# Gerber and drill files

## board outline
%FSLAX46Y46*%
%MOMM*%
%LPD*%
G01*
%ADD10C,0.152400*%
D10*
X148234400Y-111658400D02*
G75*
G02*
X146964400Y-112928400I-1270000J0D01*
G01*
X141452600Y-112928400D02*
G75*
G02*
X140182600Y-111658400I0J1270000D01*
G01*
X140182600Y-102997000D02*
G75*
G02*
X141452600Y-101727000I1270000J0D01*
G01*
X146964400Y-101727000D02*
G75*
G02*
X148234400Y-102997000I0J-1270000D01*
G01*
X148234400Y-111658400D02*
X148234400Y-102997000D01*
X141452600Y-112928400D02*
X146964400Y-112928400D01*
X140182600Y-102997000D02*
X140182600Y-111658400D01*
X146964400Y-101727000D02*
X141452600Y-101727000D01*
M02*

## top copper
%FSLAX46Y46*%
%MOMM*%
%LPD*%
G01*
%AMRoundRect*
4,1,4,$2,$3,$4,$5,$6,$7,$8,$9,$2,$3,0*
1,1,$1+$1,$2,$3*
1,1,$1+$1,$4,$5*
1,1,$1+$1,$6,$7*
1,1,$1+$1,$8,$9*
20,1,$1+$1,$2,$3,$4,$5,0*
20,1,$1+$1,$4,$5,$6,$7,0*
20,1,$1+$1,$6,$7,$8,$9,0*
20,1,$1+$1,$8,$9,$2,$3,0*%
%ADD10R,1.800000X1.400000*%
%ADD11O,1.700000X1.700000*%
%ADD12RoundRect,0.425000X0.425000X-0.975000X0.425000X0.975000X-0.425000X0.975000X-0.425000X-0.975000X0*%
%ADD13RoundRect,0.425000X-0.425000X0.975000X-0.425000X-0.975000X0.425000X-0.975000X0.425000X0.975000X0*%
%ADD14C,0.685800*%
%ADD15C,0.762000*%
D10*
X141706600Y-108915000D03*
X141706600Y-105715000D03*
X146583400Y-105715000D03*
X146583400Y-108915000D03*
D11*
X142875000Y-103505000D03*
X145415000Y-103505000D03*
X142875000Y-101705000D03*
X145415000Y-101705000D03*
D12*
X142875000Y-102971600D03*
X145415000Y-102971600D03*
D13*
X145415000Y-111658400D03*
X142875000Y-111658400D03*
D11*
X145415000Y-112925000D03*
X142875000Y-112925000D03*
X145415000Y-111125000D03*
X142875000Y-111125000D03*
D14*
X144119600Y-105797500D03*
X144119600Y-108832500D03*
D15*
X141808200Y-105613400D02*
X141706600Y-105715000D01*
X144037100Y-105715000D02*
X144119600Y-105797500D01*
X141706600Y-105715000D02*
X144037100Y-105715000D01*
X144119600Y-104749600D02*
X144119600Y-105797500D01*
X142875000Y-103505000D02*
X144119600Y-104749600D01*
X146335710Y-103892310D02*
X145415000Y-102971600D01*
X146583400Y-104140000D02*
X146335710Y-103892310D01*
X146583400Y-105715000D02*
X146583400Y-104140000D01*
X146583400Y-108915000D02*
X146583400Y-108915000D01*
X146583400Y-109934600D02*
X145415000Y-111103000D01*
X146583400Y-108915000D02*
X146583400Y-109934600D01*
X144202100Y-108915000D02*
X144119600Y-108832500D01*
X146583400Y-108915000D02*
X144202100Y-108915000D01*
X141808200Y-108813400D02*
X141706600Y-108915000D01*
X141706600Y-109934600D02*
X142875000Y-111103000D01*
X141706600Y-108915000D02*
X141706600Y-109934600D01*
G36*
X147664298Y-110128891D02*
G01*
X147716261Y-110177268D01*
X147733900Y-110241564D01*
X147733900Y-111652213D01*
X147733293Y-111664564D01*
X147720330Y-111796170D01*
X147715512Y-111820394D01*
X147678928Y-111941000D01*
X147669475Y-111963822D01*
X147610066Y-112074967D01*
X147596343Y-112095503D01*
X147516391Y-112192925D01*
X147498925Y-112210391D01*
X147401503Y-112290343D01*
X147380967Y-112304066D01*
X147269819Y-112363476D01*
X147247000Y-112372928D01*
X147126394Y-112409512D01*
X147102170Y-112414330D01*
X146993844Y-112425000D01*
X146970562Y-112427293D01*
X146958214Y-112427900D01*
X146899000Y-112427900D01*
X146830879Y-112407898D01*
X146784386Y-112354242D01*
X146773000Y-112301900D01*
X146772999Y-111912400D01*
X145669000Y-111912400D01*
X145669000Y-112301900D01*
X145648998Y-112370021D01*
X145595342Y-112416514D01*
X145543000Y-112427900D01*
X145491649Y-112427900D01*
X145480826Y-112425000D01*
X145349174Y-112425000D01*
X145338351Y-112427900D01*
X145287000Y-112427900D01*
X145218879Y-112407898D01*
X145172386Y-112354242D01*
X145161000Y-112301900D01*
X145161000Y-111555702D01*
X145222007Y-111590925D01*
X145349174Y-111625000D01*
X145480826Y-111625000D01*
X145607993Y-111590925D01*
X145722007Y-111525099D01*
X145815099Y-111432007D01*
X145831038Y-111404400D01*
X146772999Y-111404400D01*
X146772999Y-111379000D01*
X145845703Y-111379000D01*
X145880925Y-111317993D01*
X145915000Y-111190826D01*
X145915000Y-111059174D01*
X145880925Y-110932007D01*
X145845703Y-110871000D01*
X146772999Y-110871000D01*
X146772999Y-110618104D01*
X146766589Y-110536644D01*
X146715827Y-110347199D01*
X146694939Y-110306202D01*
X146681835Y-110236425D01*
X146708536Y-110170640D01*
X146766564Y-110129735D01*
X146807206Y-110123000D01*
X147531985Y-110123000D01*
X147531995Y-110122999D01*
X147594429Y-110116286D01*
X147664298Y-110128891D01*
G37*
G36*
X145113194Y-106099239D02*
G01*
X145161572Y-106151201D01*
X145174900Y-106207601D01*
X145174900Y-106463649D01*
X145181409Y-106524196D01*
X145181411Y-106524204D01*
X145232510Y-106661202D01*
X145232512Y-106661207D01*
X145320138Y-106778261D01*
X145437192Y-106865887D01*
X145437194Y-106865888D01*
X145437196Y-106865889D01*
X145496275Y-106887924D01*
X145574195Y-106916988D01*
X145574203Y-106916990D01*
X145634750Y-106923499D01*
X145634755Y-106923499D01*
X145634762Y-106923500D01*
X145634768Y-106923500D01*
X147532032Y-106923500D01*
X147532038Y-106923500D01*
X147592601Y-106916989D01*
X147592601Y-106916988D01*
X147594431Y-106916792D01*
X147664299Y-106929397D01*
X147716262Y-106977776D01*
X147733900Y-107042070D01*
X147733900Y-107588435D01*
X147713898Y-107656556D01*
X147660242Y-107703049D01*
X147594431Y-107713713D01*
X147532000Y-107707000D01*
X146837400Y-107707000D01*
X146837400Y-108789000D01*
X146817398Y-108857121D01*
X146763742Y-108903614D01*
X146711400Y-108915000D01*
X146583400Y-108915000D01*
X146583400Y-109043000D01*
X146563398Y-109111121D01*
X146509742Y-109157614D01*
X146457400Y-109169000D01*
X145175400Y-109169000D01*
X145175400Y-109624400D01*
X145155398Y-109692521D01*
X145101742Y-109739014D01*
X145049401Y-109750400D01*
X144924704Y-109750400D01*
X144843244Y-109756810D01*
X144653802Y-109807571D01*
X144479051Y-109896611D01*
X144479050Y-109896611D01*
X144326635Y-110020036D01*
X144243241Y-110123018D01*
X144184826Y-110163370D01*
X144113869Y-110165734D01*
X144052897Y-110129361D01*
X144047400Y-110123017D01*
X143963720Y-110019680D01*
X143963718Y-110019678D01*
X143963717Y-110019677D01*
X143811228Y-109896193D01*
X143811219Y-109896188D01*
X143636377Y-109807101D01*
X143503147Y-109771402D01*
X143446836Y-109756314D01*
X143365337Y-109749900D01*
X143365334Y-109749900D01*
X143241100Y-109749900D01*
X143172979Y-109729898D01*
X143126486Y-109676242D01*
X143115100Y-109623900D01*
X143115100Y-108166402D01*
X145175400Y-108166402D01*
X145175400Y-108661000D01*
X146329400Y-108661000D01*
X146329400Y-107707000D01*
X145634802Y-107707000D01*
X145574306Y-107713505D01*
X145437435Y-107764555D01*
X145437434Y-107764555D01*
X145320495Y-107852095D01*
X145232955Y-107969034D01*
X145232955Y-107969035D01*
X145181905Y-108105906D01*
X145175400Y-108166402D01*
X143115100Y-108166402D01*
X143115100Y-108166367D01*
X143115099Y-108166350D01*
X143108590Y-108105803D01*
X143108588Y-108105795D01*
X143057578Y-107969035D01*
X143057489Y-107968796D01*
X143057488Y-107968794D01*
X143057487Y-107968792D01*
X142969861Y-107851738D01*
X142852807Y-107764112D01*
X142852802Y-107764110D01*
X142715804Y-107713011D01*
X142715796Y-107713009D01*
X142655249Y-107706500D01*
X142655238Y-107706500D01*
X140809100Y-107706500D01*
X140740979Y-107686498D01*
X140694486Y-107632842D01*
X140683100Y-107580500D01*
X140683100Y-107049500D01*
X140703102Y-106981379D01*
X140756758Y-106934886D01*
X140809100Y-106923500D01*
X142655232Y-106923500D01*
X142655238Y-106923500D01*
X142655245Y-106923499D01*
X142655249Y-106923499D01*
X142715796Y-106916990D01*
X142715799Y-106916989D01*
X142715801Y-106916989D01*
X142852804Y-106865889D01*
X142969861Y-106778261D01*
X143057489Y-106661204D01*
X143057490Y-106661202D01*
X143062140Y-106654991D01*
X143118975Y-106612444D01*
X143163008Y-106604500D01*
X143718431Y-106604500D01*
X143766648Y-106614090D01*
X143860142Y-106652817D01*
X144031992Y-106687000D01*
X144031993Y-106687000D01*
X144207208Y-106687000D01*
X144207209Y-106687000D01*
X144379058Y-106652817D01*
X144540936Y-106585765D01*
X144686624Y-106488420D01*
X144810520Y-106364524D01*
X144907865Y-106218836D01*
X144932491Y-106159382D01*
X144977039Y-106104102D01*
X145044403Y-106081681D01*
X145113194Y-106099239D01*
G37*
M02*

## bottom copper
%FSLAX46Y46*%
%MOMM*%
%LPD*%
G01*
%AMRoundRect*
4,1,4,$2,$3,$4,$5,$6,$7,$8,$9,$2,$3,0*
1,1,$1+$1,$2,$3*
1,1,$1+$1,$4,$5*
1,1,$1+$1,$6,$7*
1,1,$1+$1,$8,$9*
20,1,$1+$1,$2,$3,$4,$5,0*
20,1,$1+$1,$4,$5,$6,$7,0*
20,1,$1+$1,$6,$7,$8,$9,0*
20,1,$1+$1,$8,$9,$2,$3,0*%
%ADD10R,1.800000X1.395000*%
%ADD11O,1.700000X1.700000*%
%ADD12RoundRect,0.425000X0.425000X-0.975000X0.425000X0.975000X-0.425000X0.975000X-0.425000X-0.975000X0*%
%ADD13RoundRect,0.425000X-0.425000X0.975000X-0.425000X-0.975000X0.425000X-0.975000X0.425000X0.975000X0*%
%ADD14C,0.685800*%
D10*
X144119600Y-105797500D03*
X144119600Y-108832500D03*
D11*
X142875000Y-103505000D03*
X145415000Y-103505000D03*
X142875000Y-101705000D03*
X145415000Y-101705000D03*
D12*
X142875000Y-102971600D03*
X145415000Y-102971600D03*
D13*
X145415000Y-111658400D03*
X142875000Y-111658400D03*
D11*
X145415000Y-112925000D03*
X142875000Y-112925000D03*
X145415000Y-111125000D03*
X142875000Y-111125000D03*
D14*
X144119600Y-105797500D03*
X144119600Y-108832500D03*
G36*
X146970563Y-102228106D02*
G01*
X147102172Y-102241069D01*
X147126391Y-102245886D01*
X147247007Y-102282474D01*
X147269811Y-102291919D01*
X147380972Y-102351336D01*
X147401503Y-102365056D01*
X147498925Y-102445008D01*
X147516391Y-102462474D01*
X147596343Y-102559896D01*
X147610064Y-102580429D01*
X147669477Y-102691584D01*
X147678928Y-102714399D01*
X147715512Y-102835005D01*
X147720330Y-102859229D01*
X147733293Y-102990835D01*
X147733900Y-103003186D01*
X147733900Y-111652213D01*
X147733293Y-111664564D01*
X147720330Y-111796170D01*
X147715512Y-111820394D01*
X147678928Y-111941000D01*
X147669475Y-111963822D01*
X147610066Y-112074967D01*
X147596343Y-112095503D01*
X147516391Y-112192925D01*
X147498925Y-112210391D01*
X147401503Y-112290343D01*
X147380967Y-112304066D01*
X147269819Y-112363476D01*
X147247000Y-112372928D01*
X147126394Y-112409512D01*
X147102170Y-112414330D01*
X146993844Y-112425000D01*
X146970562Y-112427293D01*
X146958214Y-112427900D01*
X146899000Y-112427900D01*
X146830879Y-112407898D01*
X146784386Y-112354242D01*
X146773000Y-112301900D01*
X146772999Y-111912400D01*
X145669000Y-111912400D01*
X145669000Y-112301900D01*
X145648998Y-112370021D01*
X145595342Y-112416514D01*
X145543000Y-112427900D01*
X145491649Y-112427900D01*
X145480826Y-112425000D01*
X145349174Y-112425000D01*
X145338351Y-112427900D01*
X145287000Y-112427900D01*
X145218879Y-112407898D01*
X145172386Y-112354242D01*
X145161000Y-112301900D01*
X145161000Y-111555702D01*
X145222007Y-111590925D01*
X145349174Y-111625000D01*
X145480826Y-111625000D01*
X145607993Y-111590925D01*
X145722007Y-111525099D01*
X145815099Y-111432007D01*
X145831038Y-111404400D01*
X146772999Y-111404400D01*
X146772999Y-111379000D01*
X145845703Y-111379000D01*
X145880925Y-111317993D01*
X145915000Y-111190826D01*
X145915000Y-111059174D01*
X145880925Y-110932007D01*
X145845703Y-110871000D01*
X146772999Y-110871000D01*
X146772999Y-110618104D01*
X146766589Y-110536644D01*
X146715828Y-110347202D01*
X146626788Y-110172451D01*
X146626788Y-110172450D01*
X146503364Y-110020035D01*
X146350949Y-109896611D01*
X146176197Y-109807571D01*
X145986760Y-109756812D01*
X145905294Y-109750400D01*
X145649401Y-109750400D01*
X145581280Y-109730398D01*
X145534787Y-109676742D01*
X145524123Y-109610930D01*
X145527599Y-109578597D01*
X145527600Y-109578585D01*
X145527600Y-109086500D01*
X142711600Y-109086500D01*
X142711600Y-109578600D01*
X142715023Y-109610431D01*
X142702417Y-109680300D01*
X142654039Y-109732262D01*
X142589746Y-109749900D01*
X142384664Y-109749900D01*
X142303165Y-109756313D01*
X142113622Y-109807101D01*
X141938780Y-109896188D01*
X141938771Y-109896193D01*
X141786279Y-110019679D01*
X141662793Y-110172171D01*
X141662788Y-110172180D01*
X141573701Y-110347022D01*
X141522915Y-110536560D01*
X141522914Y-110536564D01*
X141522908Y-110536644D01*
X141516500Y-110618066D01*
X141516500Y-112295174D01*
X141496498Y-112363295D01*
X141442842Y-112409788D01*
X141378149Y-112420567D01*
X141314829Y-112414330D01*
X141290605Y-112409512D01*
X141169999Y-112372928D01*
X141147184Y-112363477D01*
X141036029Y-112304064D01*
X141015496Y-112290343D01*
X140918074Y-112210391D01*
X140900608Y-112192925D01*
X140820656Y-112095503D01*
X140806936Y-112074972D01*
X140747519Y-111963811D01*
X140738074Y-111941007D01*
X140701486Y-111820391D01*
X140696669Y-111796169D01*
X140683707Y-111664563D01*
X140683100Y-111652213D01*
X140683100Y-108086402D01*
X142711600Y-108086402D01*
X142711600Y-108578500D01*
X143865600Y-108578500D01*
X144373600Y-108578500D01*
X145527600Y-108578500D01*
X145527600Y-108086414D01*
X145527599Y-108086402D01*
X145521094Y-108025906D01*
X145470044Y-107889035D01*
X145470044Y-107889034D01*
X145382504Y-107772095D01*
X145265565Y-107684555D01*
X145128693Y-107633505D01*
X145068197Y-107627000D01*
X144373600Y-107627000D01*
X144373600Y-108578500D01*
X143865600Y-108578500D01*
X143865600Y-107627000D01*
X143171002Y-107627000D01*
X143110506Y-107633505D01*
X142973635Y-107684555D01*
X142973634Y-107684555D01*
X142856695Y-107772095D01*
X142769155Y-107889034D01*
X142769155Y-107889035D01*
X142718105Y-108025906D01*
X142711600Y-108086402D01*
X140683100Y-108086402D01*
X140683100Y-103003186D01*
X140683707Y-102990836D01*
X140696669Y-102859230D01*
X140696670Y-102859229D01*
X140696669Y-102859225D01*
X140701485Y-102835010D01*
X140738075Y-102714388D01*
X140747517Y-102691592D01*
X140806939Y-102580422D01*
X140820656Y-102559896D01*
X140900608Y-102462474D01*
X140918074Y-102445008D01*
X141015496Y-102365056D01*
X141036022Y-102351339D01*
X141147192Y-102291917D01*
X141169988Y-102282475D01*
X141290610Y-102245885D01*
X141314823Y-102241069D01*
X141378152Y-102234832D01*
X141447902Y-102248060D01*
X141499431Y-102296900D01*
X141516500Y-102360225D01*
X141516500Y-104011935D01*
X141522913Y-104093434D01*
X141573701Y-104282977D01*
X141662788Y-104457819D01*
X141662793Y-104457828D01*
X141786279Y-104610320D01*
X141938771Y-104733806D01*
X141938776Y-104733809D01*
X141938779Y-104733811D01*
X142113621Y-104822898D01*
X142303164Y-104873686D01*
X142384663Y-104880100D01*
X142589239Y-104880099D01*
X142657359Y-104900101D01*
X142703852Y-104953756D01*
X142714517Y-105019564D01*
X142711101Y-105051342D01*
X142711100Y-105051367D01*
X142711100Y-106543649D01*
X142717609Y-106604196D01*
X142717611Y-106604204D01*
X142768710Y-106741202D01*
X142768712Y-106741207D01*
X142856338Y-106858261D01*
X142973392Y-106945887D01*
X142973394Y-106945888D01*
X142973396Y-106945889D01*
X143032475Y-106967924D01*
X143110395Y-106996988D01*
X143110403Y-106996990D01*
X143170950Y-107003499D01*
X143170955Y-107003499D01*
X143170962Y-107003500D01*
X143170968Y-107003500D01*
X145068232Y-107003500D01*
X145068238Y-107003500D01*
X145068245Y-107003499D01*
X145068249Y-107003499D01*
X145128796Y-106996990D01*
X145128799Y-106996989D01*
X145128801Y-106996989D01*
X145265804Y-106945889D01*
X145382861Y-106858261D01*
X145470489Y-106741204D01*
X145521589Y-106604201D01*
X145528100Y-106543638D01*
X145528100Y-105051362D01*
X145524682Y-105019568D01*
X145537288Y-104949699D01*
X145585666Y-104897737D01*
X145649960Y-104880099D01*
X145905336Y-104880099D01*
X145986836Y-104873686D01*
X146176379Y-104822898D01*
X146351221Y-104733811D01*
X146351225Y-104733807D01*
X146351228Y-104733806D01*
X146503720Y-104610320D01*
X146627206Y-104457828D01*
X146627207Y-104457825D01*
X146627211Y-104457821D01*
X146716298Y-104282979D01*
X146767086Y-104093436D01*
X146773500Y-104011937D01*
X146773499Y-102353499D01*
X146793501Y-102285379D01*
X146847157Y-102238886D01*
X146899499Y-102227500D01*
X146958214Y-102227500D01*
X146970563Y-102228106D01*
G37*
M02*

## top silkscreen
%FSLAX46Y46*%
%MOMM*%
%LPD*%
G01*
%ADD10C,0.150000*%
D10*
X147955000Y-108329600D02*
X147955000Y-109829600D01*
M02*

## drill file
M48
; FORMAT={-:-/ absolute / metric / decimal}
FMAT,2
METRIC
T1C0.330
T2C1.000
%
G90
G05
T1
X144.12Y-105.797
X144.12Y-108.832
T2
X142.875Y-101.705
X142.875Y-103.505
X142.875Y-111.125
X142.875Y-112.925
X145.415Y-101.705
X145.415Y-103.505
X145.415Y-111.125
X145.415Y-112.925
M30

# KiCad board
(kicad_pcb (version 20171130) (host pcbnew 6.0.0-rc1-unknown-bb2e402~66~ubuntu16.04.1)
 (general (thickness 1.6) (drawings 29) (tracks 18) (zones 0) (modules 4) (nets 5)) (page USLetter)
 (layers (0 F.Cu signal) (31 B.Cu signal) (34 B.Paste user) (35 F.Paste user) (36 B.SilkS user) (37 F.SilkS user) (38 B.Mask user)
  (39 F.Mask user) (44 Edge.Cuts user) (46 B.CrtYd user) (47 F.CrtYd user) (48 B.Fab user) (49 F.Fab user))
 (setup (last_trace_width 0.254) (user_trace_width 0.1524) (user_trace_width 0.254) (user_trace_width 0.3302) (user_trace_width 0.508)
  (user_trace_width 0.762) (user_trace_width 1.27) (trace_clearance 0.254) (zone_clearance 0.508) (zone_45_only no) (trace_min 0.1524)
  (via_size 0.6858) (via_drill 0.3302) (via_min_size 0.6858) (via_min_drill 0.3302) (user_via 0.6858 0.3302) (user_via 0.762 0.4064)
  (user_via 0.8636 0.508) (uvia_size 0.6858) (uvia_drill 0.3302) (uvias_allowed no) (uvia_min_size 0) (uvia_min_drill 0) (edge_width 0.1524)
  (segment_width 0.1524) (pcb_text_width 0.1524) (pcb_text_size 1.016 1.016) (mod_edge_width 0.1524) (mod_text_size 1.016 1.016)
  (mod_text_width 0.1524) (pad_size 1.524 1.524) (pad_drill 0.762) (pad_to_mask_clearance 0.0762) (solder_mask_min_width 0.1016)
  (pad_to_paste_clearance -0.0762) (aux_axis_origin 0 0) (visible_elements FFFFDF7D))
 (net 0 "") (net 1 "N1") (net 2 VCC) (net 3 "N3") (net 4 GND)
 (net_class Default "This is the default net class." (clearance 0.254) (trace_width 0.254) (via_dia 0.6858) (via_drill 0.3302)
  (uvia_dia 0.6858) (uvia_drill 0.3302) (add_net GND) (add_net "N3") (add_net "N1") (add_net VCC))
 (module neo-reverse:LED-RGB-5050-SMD (layer F.Cu) (at 144.145 107.315)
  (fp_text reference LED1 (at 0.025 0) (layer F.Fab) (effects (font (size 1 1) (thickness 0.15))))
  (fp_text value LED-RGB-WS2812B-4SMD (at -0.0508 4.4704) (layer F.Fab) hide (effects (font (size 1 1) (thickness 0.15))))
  (fp_line (start 3.81 1.0146) (end 3.81 2.5146) (layer F.SilkS) (width 0.15))
  (pad 4 smd rect (at -2.4384 1.6) (size 1.8 1.4) (layers F.Cu F.Paste F.Mask) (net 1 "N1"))
  (pad 3 smd rect (at -2.4384 -1.6) (size 1.8 1.4) (layers F.Cu F.Paste F.Mask) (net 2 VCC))
  (pad 2 smd rect (at 2.4384 -1.6) (size 1.8 1.4) (layers F.Cu F.Paste F.Mask) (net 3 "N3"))
  (pad 1 smd rect (at 2.4384 1.6) (size 1.8 1.4) (layers F.Cu F.Paste F.Mask) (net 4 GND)))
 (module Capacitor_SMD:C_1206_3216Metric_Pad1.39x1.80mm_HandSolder (layer B.Cu) (at 144.1196 107.315 270)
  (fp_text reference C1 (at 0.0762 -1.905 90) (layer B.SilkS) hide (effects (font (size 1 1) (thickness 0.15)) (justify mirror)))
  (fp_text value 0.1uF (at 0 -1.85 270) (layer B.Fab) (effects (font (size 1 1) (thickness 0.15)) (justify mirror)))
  (pad 1 smd rect (at -1.5175 0 270) (size 1.395 1.8) (layers B.Cu B.Paste B.Mask) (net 2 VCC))
  (pad 2 smd rect (at 1.5175 0 270) (size 1.395 1.8) (layers B.Cu B.Paste B.Mask) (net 4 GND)))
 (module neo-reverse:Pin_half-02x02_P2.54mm (layer F.Cu) (at 142.875 103.505 90)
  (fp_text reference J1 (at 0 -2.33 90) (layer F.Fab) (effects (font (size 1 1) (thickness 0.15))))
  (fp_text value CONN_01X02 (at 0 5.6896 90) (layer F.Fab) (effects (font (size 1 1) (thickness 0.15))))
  (pad 1 thru_hole oval (at 0 0 90) (size 1.7 1.7) (drill 1) (layers *.Cu *.Mask) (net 2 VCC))
  (pad 2 thru_hole oval (at 0 2.54 90) (size 1.7 1.7) (drill 1) (layers *.Cu *.Mask) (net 3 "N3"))
  (pad 1 thru_hole oval (at 1.8 0 90) (size 1.7 1.7) (drill 1) (layers *.Cu *.Mask) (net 2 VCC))
  (pad 2 thru_hole oval (at 1.8 2.54 90) (size 1.7 1.7) (drill 1) (layers *.Cu *.Mask) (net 3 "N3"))
  (pad 1 smd roundrect (at 0.5334 0 90) (size 2.8 1.7) (layers F.Cu F.Mask) (roundrect_rratio 0.25) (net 2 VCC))
  (pad 1 smd roundrect (at 0.5334 0 90) (size 2.8 1.7) (layers B.Cu B.Mask) (roundrect_rratio 0.25) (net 2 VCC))
  (pad 2 smd roundrect (at 0.5334 2.54 90) (size 2.8 1.7) (layers F.Cu F.Mask) (roundrect_rratio 0.25) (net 3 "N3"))
  (pad 2 smd roundrect (at 0.5334 2.54 90) (size 2.8 1.7) (layers B.Cu B.Mask) (roundrect_rratio 0.25) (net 3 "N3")))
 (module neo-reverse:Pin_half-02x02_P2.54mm (layer B.Cu) (at 142.875 111.125 270)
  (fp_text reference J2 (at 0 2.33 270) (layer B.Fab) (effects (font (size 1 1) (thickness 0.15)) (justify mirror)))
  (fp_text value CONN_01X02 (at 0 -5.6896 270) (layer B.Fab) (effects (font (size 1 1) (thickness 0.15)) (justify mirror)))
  (pad 2 smd roundrect (at 0.5334 -2.54 270) (size 2.8 1.7) (layers F.Cu F.Mask) (roundrect_rratio 0.25) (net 4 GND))
  (pad 2 smd roundrect (at 0.5334 -2.54 270) (size 2.8 1.7) (layers B.Cu B.Mask) (roundrect_rratio 0.25) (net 4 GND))
  (pad 1 smd roundrect (at 0.5334 0 270) (size 2.8 1.7) (layers F.Cu F.Mask) (roundrect_rratio 0.25) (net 1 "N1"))
  (pad 1 smd roundrect (at 0.5334 0 270) (size 2.8 1.7) (layers B.Cu B.Mask) (roundrect_rratio 0.25) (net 1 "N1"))
  (pad 2 thru_hole oval (at 1.8 -2.54 270) (size 1.7 1.7) (drill 1) (layers *.Cu *.Mask) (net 4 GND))
  (pad 1 thru_hole oval (at 1.8 0 270) (size 1.7 1.7) (drill 1) (layers *.Cu *.Mask) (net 1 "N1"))
  (pad 2 thru_hole oval (at 0 -2.54 270) (size 1.7 1.7) (drill 1) (layers *.Cu *.Mask) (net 4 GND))
  (pad 1 thru_hole oval (at 0 0 270) (size 1.7 1.7) (drill 1) (layers *.Cu *.Mask) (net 1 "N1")))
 (gr_arc (start 146.9644 111.6584) (end 146.9644 112.9284) (angle -90) (layer Edge.Cuts) (width 0.1524))
 (gr_arc (start 141.4526 111.6584) (end 140.1826 111.6584) (angle -90) (layer Edge.Cuts) (width 0.1524))
 (gr_arc (start 141.4526 102.997) (end 141.4526 101.727) (angle -90) (layer Edge.Cuts) (width 0.1524))
 (gr_arc (start 146.9644 102.997) (end 148.2344 102.997) (angle -90) (layer Edge.Cuts) (width 0.1524))
 (gr_line (start 148.2344 111.6584) (end 148.2344 102.997) (layer Edge.Cuts) (width 0.1524))
 (gr_line (start 141.4526 112.9284) (end 146.9644 112.9284) (layer Edge.Cuts) (width 0.1524))
 (gr_line (start 140.1826 102.997) (end 140.1826 111.6584) (layer Edge.Cuts) (width 0.1524))
 (gr_line (start 146.9644 101.727) (end 141.4526 101.727) (layer Edge.Cuts) (width 0.1524))
 (segment (start 141.8082 105.6134) (end 141.7066 105.715) (width 0.762) (layer F.Cu) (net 2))
 (segment (start 144.0371 105.715) (end 144.1196 105.7975) (width 0.762) (layer F.Cu) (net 2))
 (via (at 144.1196 105.7975) (size 0.6858) (drill 0.3302) (layers F.Cu B.Cu) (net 2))
 (segment (start 141.7066 105.715) (end 144.0371 105.715) (width 0.762) (layer F.Cu) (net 2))
 (segment (start 144.1196 104.7496) (end 144.1196 105.7975) (width 0.762) (layer F.Cu) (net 2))
 (segment (start 142.875 103.505) (end 144.1196 104.7496) (width 0.762) (layer F.Cu) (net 2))
 (segment (start 146.33571 103.89231) (end 145.415 102.9716) (width 0.762) (layer F.Cu) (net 3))
 (segment (start 146.5834 104.14) (end 146.33571 103.89231) (width 0.762) (layer F.Cu) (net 3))
 (segment (start 146.5834 105.715) (end 146.5834 104.14) (width 0.762) (layer F.Cu) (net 3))
 (segment (start 146.5834 108.915) (end 146.5834 108.915) (width 0.762) (layer F.Cu) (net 4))
 (segment (start 146.5834 109.9346) (end 145.415 111.103) (width 0.762) (layer F.Cu) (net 4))
 (segment (start 146.5834 108.915) (end 146.5834 109.9346) (width 0.762) (layer F.Cu) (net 4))
 (segment (start 144.2021 108.915) (end 144.1196 108.8325) (width 0.762) (layer F.Cu) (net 4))
 (via (at 144.1196 108.8325) (size 0.6858) (drill 0.3302) (layers F.Cu B.Cu) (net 4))
 (segment (start 146.5834 108.915) (end 144.2021 108.915) (width 0.762) (layer F.Cu) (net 4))
 (segment (start 141.8082 108.8134) (end 141.7066 108.915) (width 0.762) (layer F.Cu) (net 1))
 (segment (start 141.7066 109.9346) (end 142.875 111.103) (width 0.762) (layer F.Cu) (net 1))
 (segment (start 141.7066 108.915) (end 141.7066 109.9346) (width 0.762) (layer F.Cu) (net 1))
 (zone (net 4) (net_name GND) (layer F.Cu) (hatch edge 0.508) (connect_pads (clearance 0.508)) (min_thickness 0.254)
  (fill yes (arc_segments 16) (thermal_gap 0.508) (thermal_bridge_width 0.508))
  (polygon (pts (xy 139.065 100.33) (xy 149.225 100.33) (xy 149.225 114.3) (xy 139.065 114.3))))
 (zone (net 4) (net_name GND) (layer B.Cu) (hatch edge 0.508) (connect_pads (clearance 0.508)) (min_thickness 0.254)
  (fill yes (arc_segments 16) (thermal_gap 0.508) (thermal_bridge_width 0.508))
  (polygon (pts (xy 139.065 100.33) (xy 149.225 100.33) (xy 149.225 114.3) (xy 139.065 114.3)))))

